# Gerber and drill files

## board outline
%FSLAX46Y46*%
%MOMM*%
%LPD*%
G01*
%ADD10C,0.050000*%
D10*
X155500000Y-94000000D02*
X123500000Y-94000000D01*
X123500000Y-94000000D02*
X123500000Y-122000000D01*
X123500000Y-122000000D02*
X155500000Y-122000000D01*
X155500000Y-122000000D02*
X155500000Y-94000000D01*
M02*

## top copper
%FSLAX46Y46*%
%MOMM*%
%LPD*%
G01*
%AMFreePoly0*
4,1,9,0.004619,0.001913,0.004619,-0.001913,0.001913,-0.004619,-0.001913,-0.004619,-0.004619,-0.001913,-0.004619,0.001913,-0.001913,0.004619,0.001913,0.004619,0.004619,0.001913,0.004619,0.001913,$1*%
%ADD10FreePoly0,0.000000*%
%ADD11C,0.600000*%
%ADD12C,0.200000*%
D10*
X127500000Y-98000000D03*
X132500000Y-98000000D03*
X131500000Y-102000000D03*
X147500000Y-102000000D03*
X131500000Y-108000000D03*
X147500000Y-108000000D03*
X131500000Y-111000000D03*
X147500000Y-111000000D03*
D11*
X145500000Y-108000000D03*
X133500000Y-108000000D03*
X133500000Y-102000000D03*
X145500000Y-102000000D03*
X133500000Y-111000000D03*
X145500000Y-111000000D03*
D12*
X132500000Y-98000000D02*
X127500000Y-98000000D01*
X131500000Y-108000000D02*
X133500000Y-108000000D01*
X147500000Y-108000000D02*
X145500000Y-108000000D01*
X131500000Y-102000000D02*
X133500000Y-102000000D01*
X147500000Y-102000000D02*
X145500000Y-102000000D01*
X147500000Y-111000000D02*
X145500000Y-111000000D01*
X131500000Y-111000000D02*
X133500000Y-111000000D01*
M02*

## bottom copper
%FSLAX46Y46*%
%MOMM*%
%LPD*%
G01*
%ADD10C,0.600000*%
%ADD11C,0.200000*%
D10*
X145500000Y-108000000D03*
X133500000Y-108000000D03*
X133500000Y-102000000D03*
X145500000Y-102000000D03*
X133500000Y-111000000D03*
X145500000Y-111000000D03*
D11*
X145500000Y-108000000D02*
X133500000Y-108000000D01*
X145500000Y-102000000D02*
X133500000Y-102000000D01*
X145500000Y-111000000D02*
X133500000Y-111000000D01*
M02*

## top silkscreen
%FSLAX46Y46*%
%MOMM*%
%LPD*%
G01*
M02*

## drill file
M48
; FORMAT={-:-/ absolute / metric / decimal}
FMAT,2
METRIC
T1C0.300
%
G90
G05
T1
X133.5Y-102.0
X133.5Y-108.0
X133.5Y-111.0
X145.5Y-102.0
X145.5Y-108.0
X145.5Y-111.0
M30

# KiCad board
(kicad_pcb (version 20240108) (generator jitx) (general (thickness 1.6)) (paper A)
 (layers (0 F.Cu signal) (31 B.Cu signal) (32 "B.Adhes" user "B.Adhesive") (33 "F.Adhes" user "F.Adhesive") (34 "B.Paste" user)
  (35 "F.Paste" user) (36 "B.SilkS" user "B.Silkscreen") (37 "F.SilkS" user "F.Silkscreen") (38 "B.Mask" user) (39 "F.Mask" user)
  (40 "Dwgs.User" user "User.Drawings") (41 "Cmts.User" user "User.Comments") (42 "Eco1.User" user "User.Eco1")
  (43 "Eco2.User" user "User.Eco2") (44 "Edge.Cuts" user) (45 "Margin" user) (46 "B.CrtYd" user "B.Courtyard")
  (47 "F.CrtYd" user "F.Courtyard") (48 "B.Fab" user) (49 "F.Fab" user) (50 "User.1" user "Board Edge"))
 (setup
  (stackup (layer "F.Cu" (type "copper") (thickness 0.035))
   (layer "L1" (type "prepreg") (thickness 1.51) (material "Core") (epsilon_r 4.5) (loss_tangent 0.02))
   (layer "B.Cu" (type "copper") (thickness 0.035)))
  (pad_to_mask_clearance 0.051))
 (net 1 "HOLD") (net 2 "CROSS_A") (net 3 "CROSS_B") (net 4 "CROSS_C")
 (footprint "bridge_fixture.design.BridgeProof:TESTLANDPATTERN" (layer F.Cu) (at 127.5 98.0 0.0)
  (pad p smd custom (at 0.0 0.0 0.0) (size 0.01 0.01) (options (clearance outline) (anchor circle)) (primitives) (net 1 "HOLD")
   (layers F.Cu))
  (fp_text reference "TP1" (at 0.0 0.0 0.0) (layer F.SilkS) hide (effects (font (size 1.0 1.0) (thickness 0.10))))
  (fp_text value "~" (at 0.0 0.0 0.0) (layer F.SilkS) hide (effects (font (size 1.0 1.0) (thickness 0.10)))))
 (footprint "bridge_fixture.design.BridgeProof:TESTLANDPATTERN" (layer F.Cu) (at 132.5 98.0 0.0)
  (pad p smd custom (at 0.0 0.0 0.0) (size 0.01 0.01) (options (clearance outline) (anchor circle)) (primitives) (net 1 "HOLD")
   (layers F.Cu))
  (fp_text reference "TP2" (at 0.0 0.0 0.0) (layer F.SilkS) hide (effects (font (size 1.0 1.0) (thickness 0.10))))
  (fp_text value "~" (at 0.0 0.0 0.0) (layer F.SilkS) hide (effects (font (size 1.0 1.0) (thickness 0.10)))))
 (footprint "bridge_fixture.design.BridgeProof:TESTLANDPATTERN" (layer F.Cu) (at 131.5 102.0 0.0)
  (pad p smd custom (at 0.0 0.0 0.0) (size 0.01 0.01) (options (clearance outline) (anchor circle)) (primitives) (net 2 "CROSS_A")
   (layers F.Cu))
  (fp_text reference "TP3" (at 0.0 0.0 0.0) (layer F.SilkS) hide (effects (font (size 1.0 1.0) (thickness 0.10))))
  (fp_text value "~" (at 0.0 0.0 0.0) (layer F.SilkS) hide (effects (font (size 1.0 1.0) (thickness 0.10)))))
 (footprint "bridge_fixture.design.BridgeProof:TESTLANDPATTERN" (layer F.Cu) (at 147.5 102.0 0.0)
  (pad p smd custom (at 0.0 0.0 0.0) (size 0.01 0.01) (options (clearance outline) (anchor circle)) (primitives) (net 2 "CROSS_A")
   (layers F.Cu))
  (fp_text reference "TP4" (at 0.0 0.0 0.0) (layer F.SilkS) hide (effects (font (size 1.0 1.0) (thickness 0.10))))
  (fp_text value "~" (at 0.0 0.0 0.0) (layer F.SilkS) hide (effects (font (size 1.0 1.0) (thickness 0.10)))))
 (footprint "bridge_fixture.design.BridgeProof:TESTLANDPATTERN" (layer F.Cu) (at 131.5 108.0 0.0)
  (pad p smd custom (at 0.0 0.0 0.0) (size 0.01 0.01) (options (clearance outline) (anchor circle)) (primitives) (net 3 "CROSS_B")
   (layers F.Cu))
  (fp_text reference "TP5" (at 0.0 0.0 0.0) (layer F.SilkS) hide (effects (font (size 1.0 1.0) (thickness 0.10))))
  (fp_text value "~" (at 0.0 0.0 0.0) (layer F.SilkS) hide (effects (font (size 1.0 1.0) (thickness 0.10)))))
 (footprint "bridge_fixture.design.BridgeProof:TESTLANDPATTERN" (layer F.Cu) (at 147.5 108.0 0.0)
  (pad p smd custom (at 0.0 0.0 0.0) (size 0.01 0.01) (options (clearance outline) (anchor circle)) (primitives) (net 3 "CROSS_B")
   (layers F.Cu))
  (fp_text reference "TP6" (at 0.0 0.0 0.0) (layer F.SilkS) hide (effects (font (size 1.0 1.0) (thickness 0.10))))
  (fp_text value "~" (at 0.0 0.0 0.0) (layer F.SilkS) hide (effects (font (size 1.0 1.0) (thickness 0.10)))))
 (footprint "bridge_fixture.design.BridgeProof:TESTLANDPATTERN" (layer F.Cu) (at 131.5 111.0 0.0)
  (pad p smd custom (at 0.0 0.0 0.0) (size 0.01 0.01) (options (clearance outline) (anchor circle)) (primitives) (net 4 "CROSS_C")
   (layers F.Cu))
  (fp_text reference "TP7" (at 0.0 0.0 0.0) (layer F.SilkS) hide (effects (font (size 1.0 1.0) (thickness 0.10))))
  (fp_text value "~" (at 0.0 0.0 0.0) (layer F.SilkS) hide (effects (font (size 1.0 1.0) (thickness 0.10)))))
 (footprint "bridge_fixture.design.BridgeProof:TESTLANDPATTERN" (layer F.Cu) (at 147.5 111.0 0.0)
  (pad p smd custom (at 0.0 0.0 0.0) (size 0.01 0.01) (options (clearance outline) (anchor circle)) (primitives) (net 4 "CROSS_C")
   (layers F.Cu))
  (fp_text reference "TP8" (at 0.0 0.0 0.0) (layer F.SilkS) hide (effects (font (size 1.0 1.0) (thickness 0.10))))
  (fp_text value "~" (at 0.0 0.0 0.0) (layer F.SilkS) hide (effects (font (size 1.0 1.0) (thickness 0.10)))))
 (segment (start 132.5 98.0) (end 127.5 98.0) (layer F.Cu) (width 0.2) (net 1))
 (segment (start 145.500000001462 108.000000001315) (end 133.499999998538 108.000000001315) (layer B.Cu) (width 0.2) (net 3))
 (segment (start 131.5 108.0) (end 133.499999998538 108.000000001315) (layer F.Cu) (width 0.2) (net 3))
 (segment (start 147.5 108.0) (end 145.500000001462 108.000000001315) (layer F.Cu) (width 0.2) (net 3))
 (segment (start 145.500000004939 101.999999997439) (end 133.499999995061 101.999999997439) (layer B.Cu) (width 0.2) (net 2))
 (segment (start 131.5 102.0) (end 133.499999995061 101.999999997439) (layer F.Cu) (width 0.2) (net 2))
 (segment (start 147.5 102.0) (end 145.500000004939 101.999999997439) (layer F.Cu) (width 0.2) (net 2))
 (segment (start 145.500000001462 110.999999998685) (end 133.499999998538 110.999999998685) (layer B.Cu) (width 0.2) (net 4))
 (segment (start 147.5 111.0) (end 145.500000001462 110.999999998685) (layer F.Cu) (width 0.2) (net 4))
 (segment (start 131.5 111.0) (end 133.499999998538 110.999999998685) (layer F.Cu) (width 0.2) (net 4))
 (via (at 145.500000001462 108.000000001315) (size 0.6) (drill 0.3) (layers F.Cu B.Cu) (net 3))
 (via (at 133.499999998538 108.000000001315) (size 0.6) (drill 0.3) (layers F.Cu B.Cu) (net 3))
 (via (at 133.499999995061 101.999999997439) (size 0.6) (drill 0.3) (layers F.Cu B.Cu) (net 2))
 (via (at 145.500000004939 101.999999997439) (size 0.6) (drill 0.3) (layers F.Cu B.Cu) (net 2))
 (via (at 133.499999998538 110.999999998685) (size 0.6) (drill 0.3) (layers F.Cu B.Cu) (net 4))
 (via (at 145.500000001462 110.999999998685) (size 0.6) (drill 0.3) (layers F.Cu B.Cu) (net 4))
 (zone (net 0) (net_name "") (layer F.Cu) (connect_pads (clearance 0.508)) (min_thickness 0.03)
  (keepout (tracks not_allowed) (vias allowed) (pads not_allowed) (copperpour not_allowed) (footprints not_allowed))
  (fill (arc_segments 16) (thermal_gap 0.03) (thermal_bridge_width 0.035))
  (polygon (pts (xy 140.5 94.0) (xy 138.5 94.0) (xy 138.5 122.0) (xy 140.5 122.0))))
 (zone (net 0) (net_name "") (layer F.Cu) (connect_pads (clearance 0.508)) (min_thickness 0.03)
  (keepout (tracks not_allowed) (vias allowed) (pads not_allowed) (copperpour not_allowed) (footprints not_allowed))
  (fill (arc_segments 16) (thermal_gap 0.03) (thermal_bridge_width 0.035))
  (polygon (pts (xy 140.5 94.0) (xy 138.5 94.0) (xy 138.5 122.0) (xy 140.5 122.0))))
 (gr_line (start 155.5 94.0) (end 123.5 94.0) (layer Edge.Cuts) (stroke (width 0.05) (type solid)))
 (gr_line (start 123.5 94.0) (end 123.5 122.0) (layer Edge.Cuts) (stroke (width 0.05) (type solid)))
 (gr_line (start 123.5 122.0) (end 155.5 122.0) (layer Edge.Cuts) (stroke (width 0.05) (type solid)))
 (gr_line (start 155.5 122.0) (end 155.5 94.0) (layer Edge.Cuts) (stroke (width 0.05) (type solid)))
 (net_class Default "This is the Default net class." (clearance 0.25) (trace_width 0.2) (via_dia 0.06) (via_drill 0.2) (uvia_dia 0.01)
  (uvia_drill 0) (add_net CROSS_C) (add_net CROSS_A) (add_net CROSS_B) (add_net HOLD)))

